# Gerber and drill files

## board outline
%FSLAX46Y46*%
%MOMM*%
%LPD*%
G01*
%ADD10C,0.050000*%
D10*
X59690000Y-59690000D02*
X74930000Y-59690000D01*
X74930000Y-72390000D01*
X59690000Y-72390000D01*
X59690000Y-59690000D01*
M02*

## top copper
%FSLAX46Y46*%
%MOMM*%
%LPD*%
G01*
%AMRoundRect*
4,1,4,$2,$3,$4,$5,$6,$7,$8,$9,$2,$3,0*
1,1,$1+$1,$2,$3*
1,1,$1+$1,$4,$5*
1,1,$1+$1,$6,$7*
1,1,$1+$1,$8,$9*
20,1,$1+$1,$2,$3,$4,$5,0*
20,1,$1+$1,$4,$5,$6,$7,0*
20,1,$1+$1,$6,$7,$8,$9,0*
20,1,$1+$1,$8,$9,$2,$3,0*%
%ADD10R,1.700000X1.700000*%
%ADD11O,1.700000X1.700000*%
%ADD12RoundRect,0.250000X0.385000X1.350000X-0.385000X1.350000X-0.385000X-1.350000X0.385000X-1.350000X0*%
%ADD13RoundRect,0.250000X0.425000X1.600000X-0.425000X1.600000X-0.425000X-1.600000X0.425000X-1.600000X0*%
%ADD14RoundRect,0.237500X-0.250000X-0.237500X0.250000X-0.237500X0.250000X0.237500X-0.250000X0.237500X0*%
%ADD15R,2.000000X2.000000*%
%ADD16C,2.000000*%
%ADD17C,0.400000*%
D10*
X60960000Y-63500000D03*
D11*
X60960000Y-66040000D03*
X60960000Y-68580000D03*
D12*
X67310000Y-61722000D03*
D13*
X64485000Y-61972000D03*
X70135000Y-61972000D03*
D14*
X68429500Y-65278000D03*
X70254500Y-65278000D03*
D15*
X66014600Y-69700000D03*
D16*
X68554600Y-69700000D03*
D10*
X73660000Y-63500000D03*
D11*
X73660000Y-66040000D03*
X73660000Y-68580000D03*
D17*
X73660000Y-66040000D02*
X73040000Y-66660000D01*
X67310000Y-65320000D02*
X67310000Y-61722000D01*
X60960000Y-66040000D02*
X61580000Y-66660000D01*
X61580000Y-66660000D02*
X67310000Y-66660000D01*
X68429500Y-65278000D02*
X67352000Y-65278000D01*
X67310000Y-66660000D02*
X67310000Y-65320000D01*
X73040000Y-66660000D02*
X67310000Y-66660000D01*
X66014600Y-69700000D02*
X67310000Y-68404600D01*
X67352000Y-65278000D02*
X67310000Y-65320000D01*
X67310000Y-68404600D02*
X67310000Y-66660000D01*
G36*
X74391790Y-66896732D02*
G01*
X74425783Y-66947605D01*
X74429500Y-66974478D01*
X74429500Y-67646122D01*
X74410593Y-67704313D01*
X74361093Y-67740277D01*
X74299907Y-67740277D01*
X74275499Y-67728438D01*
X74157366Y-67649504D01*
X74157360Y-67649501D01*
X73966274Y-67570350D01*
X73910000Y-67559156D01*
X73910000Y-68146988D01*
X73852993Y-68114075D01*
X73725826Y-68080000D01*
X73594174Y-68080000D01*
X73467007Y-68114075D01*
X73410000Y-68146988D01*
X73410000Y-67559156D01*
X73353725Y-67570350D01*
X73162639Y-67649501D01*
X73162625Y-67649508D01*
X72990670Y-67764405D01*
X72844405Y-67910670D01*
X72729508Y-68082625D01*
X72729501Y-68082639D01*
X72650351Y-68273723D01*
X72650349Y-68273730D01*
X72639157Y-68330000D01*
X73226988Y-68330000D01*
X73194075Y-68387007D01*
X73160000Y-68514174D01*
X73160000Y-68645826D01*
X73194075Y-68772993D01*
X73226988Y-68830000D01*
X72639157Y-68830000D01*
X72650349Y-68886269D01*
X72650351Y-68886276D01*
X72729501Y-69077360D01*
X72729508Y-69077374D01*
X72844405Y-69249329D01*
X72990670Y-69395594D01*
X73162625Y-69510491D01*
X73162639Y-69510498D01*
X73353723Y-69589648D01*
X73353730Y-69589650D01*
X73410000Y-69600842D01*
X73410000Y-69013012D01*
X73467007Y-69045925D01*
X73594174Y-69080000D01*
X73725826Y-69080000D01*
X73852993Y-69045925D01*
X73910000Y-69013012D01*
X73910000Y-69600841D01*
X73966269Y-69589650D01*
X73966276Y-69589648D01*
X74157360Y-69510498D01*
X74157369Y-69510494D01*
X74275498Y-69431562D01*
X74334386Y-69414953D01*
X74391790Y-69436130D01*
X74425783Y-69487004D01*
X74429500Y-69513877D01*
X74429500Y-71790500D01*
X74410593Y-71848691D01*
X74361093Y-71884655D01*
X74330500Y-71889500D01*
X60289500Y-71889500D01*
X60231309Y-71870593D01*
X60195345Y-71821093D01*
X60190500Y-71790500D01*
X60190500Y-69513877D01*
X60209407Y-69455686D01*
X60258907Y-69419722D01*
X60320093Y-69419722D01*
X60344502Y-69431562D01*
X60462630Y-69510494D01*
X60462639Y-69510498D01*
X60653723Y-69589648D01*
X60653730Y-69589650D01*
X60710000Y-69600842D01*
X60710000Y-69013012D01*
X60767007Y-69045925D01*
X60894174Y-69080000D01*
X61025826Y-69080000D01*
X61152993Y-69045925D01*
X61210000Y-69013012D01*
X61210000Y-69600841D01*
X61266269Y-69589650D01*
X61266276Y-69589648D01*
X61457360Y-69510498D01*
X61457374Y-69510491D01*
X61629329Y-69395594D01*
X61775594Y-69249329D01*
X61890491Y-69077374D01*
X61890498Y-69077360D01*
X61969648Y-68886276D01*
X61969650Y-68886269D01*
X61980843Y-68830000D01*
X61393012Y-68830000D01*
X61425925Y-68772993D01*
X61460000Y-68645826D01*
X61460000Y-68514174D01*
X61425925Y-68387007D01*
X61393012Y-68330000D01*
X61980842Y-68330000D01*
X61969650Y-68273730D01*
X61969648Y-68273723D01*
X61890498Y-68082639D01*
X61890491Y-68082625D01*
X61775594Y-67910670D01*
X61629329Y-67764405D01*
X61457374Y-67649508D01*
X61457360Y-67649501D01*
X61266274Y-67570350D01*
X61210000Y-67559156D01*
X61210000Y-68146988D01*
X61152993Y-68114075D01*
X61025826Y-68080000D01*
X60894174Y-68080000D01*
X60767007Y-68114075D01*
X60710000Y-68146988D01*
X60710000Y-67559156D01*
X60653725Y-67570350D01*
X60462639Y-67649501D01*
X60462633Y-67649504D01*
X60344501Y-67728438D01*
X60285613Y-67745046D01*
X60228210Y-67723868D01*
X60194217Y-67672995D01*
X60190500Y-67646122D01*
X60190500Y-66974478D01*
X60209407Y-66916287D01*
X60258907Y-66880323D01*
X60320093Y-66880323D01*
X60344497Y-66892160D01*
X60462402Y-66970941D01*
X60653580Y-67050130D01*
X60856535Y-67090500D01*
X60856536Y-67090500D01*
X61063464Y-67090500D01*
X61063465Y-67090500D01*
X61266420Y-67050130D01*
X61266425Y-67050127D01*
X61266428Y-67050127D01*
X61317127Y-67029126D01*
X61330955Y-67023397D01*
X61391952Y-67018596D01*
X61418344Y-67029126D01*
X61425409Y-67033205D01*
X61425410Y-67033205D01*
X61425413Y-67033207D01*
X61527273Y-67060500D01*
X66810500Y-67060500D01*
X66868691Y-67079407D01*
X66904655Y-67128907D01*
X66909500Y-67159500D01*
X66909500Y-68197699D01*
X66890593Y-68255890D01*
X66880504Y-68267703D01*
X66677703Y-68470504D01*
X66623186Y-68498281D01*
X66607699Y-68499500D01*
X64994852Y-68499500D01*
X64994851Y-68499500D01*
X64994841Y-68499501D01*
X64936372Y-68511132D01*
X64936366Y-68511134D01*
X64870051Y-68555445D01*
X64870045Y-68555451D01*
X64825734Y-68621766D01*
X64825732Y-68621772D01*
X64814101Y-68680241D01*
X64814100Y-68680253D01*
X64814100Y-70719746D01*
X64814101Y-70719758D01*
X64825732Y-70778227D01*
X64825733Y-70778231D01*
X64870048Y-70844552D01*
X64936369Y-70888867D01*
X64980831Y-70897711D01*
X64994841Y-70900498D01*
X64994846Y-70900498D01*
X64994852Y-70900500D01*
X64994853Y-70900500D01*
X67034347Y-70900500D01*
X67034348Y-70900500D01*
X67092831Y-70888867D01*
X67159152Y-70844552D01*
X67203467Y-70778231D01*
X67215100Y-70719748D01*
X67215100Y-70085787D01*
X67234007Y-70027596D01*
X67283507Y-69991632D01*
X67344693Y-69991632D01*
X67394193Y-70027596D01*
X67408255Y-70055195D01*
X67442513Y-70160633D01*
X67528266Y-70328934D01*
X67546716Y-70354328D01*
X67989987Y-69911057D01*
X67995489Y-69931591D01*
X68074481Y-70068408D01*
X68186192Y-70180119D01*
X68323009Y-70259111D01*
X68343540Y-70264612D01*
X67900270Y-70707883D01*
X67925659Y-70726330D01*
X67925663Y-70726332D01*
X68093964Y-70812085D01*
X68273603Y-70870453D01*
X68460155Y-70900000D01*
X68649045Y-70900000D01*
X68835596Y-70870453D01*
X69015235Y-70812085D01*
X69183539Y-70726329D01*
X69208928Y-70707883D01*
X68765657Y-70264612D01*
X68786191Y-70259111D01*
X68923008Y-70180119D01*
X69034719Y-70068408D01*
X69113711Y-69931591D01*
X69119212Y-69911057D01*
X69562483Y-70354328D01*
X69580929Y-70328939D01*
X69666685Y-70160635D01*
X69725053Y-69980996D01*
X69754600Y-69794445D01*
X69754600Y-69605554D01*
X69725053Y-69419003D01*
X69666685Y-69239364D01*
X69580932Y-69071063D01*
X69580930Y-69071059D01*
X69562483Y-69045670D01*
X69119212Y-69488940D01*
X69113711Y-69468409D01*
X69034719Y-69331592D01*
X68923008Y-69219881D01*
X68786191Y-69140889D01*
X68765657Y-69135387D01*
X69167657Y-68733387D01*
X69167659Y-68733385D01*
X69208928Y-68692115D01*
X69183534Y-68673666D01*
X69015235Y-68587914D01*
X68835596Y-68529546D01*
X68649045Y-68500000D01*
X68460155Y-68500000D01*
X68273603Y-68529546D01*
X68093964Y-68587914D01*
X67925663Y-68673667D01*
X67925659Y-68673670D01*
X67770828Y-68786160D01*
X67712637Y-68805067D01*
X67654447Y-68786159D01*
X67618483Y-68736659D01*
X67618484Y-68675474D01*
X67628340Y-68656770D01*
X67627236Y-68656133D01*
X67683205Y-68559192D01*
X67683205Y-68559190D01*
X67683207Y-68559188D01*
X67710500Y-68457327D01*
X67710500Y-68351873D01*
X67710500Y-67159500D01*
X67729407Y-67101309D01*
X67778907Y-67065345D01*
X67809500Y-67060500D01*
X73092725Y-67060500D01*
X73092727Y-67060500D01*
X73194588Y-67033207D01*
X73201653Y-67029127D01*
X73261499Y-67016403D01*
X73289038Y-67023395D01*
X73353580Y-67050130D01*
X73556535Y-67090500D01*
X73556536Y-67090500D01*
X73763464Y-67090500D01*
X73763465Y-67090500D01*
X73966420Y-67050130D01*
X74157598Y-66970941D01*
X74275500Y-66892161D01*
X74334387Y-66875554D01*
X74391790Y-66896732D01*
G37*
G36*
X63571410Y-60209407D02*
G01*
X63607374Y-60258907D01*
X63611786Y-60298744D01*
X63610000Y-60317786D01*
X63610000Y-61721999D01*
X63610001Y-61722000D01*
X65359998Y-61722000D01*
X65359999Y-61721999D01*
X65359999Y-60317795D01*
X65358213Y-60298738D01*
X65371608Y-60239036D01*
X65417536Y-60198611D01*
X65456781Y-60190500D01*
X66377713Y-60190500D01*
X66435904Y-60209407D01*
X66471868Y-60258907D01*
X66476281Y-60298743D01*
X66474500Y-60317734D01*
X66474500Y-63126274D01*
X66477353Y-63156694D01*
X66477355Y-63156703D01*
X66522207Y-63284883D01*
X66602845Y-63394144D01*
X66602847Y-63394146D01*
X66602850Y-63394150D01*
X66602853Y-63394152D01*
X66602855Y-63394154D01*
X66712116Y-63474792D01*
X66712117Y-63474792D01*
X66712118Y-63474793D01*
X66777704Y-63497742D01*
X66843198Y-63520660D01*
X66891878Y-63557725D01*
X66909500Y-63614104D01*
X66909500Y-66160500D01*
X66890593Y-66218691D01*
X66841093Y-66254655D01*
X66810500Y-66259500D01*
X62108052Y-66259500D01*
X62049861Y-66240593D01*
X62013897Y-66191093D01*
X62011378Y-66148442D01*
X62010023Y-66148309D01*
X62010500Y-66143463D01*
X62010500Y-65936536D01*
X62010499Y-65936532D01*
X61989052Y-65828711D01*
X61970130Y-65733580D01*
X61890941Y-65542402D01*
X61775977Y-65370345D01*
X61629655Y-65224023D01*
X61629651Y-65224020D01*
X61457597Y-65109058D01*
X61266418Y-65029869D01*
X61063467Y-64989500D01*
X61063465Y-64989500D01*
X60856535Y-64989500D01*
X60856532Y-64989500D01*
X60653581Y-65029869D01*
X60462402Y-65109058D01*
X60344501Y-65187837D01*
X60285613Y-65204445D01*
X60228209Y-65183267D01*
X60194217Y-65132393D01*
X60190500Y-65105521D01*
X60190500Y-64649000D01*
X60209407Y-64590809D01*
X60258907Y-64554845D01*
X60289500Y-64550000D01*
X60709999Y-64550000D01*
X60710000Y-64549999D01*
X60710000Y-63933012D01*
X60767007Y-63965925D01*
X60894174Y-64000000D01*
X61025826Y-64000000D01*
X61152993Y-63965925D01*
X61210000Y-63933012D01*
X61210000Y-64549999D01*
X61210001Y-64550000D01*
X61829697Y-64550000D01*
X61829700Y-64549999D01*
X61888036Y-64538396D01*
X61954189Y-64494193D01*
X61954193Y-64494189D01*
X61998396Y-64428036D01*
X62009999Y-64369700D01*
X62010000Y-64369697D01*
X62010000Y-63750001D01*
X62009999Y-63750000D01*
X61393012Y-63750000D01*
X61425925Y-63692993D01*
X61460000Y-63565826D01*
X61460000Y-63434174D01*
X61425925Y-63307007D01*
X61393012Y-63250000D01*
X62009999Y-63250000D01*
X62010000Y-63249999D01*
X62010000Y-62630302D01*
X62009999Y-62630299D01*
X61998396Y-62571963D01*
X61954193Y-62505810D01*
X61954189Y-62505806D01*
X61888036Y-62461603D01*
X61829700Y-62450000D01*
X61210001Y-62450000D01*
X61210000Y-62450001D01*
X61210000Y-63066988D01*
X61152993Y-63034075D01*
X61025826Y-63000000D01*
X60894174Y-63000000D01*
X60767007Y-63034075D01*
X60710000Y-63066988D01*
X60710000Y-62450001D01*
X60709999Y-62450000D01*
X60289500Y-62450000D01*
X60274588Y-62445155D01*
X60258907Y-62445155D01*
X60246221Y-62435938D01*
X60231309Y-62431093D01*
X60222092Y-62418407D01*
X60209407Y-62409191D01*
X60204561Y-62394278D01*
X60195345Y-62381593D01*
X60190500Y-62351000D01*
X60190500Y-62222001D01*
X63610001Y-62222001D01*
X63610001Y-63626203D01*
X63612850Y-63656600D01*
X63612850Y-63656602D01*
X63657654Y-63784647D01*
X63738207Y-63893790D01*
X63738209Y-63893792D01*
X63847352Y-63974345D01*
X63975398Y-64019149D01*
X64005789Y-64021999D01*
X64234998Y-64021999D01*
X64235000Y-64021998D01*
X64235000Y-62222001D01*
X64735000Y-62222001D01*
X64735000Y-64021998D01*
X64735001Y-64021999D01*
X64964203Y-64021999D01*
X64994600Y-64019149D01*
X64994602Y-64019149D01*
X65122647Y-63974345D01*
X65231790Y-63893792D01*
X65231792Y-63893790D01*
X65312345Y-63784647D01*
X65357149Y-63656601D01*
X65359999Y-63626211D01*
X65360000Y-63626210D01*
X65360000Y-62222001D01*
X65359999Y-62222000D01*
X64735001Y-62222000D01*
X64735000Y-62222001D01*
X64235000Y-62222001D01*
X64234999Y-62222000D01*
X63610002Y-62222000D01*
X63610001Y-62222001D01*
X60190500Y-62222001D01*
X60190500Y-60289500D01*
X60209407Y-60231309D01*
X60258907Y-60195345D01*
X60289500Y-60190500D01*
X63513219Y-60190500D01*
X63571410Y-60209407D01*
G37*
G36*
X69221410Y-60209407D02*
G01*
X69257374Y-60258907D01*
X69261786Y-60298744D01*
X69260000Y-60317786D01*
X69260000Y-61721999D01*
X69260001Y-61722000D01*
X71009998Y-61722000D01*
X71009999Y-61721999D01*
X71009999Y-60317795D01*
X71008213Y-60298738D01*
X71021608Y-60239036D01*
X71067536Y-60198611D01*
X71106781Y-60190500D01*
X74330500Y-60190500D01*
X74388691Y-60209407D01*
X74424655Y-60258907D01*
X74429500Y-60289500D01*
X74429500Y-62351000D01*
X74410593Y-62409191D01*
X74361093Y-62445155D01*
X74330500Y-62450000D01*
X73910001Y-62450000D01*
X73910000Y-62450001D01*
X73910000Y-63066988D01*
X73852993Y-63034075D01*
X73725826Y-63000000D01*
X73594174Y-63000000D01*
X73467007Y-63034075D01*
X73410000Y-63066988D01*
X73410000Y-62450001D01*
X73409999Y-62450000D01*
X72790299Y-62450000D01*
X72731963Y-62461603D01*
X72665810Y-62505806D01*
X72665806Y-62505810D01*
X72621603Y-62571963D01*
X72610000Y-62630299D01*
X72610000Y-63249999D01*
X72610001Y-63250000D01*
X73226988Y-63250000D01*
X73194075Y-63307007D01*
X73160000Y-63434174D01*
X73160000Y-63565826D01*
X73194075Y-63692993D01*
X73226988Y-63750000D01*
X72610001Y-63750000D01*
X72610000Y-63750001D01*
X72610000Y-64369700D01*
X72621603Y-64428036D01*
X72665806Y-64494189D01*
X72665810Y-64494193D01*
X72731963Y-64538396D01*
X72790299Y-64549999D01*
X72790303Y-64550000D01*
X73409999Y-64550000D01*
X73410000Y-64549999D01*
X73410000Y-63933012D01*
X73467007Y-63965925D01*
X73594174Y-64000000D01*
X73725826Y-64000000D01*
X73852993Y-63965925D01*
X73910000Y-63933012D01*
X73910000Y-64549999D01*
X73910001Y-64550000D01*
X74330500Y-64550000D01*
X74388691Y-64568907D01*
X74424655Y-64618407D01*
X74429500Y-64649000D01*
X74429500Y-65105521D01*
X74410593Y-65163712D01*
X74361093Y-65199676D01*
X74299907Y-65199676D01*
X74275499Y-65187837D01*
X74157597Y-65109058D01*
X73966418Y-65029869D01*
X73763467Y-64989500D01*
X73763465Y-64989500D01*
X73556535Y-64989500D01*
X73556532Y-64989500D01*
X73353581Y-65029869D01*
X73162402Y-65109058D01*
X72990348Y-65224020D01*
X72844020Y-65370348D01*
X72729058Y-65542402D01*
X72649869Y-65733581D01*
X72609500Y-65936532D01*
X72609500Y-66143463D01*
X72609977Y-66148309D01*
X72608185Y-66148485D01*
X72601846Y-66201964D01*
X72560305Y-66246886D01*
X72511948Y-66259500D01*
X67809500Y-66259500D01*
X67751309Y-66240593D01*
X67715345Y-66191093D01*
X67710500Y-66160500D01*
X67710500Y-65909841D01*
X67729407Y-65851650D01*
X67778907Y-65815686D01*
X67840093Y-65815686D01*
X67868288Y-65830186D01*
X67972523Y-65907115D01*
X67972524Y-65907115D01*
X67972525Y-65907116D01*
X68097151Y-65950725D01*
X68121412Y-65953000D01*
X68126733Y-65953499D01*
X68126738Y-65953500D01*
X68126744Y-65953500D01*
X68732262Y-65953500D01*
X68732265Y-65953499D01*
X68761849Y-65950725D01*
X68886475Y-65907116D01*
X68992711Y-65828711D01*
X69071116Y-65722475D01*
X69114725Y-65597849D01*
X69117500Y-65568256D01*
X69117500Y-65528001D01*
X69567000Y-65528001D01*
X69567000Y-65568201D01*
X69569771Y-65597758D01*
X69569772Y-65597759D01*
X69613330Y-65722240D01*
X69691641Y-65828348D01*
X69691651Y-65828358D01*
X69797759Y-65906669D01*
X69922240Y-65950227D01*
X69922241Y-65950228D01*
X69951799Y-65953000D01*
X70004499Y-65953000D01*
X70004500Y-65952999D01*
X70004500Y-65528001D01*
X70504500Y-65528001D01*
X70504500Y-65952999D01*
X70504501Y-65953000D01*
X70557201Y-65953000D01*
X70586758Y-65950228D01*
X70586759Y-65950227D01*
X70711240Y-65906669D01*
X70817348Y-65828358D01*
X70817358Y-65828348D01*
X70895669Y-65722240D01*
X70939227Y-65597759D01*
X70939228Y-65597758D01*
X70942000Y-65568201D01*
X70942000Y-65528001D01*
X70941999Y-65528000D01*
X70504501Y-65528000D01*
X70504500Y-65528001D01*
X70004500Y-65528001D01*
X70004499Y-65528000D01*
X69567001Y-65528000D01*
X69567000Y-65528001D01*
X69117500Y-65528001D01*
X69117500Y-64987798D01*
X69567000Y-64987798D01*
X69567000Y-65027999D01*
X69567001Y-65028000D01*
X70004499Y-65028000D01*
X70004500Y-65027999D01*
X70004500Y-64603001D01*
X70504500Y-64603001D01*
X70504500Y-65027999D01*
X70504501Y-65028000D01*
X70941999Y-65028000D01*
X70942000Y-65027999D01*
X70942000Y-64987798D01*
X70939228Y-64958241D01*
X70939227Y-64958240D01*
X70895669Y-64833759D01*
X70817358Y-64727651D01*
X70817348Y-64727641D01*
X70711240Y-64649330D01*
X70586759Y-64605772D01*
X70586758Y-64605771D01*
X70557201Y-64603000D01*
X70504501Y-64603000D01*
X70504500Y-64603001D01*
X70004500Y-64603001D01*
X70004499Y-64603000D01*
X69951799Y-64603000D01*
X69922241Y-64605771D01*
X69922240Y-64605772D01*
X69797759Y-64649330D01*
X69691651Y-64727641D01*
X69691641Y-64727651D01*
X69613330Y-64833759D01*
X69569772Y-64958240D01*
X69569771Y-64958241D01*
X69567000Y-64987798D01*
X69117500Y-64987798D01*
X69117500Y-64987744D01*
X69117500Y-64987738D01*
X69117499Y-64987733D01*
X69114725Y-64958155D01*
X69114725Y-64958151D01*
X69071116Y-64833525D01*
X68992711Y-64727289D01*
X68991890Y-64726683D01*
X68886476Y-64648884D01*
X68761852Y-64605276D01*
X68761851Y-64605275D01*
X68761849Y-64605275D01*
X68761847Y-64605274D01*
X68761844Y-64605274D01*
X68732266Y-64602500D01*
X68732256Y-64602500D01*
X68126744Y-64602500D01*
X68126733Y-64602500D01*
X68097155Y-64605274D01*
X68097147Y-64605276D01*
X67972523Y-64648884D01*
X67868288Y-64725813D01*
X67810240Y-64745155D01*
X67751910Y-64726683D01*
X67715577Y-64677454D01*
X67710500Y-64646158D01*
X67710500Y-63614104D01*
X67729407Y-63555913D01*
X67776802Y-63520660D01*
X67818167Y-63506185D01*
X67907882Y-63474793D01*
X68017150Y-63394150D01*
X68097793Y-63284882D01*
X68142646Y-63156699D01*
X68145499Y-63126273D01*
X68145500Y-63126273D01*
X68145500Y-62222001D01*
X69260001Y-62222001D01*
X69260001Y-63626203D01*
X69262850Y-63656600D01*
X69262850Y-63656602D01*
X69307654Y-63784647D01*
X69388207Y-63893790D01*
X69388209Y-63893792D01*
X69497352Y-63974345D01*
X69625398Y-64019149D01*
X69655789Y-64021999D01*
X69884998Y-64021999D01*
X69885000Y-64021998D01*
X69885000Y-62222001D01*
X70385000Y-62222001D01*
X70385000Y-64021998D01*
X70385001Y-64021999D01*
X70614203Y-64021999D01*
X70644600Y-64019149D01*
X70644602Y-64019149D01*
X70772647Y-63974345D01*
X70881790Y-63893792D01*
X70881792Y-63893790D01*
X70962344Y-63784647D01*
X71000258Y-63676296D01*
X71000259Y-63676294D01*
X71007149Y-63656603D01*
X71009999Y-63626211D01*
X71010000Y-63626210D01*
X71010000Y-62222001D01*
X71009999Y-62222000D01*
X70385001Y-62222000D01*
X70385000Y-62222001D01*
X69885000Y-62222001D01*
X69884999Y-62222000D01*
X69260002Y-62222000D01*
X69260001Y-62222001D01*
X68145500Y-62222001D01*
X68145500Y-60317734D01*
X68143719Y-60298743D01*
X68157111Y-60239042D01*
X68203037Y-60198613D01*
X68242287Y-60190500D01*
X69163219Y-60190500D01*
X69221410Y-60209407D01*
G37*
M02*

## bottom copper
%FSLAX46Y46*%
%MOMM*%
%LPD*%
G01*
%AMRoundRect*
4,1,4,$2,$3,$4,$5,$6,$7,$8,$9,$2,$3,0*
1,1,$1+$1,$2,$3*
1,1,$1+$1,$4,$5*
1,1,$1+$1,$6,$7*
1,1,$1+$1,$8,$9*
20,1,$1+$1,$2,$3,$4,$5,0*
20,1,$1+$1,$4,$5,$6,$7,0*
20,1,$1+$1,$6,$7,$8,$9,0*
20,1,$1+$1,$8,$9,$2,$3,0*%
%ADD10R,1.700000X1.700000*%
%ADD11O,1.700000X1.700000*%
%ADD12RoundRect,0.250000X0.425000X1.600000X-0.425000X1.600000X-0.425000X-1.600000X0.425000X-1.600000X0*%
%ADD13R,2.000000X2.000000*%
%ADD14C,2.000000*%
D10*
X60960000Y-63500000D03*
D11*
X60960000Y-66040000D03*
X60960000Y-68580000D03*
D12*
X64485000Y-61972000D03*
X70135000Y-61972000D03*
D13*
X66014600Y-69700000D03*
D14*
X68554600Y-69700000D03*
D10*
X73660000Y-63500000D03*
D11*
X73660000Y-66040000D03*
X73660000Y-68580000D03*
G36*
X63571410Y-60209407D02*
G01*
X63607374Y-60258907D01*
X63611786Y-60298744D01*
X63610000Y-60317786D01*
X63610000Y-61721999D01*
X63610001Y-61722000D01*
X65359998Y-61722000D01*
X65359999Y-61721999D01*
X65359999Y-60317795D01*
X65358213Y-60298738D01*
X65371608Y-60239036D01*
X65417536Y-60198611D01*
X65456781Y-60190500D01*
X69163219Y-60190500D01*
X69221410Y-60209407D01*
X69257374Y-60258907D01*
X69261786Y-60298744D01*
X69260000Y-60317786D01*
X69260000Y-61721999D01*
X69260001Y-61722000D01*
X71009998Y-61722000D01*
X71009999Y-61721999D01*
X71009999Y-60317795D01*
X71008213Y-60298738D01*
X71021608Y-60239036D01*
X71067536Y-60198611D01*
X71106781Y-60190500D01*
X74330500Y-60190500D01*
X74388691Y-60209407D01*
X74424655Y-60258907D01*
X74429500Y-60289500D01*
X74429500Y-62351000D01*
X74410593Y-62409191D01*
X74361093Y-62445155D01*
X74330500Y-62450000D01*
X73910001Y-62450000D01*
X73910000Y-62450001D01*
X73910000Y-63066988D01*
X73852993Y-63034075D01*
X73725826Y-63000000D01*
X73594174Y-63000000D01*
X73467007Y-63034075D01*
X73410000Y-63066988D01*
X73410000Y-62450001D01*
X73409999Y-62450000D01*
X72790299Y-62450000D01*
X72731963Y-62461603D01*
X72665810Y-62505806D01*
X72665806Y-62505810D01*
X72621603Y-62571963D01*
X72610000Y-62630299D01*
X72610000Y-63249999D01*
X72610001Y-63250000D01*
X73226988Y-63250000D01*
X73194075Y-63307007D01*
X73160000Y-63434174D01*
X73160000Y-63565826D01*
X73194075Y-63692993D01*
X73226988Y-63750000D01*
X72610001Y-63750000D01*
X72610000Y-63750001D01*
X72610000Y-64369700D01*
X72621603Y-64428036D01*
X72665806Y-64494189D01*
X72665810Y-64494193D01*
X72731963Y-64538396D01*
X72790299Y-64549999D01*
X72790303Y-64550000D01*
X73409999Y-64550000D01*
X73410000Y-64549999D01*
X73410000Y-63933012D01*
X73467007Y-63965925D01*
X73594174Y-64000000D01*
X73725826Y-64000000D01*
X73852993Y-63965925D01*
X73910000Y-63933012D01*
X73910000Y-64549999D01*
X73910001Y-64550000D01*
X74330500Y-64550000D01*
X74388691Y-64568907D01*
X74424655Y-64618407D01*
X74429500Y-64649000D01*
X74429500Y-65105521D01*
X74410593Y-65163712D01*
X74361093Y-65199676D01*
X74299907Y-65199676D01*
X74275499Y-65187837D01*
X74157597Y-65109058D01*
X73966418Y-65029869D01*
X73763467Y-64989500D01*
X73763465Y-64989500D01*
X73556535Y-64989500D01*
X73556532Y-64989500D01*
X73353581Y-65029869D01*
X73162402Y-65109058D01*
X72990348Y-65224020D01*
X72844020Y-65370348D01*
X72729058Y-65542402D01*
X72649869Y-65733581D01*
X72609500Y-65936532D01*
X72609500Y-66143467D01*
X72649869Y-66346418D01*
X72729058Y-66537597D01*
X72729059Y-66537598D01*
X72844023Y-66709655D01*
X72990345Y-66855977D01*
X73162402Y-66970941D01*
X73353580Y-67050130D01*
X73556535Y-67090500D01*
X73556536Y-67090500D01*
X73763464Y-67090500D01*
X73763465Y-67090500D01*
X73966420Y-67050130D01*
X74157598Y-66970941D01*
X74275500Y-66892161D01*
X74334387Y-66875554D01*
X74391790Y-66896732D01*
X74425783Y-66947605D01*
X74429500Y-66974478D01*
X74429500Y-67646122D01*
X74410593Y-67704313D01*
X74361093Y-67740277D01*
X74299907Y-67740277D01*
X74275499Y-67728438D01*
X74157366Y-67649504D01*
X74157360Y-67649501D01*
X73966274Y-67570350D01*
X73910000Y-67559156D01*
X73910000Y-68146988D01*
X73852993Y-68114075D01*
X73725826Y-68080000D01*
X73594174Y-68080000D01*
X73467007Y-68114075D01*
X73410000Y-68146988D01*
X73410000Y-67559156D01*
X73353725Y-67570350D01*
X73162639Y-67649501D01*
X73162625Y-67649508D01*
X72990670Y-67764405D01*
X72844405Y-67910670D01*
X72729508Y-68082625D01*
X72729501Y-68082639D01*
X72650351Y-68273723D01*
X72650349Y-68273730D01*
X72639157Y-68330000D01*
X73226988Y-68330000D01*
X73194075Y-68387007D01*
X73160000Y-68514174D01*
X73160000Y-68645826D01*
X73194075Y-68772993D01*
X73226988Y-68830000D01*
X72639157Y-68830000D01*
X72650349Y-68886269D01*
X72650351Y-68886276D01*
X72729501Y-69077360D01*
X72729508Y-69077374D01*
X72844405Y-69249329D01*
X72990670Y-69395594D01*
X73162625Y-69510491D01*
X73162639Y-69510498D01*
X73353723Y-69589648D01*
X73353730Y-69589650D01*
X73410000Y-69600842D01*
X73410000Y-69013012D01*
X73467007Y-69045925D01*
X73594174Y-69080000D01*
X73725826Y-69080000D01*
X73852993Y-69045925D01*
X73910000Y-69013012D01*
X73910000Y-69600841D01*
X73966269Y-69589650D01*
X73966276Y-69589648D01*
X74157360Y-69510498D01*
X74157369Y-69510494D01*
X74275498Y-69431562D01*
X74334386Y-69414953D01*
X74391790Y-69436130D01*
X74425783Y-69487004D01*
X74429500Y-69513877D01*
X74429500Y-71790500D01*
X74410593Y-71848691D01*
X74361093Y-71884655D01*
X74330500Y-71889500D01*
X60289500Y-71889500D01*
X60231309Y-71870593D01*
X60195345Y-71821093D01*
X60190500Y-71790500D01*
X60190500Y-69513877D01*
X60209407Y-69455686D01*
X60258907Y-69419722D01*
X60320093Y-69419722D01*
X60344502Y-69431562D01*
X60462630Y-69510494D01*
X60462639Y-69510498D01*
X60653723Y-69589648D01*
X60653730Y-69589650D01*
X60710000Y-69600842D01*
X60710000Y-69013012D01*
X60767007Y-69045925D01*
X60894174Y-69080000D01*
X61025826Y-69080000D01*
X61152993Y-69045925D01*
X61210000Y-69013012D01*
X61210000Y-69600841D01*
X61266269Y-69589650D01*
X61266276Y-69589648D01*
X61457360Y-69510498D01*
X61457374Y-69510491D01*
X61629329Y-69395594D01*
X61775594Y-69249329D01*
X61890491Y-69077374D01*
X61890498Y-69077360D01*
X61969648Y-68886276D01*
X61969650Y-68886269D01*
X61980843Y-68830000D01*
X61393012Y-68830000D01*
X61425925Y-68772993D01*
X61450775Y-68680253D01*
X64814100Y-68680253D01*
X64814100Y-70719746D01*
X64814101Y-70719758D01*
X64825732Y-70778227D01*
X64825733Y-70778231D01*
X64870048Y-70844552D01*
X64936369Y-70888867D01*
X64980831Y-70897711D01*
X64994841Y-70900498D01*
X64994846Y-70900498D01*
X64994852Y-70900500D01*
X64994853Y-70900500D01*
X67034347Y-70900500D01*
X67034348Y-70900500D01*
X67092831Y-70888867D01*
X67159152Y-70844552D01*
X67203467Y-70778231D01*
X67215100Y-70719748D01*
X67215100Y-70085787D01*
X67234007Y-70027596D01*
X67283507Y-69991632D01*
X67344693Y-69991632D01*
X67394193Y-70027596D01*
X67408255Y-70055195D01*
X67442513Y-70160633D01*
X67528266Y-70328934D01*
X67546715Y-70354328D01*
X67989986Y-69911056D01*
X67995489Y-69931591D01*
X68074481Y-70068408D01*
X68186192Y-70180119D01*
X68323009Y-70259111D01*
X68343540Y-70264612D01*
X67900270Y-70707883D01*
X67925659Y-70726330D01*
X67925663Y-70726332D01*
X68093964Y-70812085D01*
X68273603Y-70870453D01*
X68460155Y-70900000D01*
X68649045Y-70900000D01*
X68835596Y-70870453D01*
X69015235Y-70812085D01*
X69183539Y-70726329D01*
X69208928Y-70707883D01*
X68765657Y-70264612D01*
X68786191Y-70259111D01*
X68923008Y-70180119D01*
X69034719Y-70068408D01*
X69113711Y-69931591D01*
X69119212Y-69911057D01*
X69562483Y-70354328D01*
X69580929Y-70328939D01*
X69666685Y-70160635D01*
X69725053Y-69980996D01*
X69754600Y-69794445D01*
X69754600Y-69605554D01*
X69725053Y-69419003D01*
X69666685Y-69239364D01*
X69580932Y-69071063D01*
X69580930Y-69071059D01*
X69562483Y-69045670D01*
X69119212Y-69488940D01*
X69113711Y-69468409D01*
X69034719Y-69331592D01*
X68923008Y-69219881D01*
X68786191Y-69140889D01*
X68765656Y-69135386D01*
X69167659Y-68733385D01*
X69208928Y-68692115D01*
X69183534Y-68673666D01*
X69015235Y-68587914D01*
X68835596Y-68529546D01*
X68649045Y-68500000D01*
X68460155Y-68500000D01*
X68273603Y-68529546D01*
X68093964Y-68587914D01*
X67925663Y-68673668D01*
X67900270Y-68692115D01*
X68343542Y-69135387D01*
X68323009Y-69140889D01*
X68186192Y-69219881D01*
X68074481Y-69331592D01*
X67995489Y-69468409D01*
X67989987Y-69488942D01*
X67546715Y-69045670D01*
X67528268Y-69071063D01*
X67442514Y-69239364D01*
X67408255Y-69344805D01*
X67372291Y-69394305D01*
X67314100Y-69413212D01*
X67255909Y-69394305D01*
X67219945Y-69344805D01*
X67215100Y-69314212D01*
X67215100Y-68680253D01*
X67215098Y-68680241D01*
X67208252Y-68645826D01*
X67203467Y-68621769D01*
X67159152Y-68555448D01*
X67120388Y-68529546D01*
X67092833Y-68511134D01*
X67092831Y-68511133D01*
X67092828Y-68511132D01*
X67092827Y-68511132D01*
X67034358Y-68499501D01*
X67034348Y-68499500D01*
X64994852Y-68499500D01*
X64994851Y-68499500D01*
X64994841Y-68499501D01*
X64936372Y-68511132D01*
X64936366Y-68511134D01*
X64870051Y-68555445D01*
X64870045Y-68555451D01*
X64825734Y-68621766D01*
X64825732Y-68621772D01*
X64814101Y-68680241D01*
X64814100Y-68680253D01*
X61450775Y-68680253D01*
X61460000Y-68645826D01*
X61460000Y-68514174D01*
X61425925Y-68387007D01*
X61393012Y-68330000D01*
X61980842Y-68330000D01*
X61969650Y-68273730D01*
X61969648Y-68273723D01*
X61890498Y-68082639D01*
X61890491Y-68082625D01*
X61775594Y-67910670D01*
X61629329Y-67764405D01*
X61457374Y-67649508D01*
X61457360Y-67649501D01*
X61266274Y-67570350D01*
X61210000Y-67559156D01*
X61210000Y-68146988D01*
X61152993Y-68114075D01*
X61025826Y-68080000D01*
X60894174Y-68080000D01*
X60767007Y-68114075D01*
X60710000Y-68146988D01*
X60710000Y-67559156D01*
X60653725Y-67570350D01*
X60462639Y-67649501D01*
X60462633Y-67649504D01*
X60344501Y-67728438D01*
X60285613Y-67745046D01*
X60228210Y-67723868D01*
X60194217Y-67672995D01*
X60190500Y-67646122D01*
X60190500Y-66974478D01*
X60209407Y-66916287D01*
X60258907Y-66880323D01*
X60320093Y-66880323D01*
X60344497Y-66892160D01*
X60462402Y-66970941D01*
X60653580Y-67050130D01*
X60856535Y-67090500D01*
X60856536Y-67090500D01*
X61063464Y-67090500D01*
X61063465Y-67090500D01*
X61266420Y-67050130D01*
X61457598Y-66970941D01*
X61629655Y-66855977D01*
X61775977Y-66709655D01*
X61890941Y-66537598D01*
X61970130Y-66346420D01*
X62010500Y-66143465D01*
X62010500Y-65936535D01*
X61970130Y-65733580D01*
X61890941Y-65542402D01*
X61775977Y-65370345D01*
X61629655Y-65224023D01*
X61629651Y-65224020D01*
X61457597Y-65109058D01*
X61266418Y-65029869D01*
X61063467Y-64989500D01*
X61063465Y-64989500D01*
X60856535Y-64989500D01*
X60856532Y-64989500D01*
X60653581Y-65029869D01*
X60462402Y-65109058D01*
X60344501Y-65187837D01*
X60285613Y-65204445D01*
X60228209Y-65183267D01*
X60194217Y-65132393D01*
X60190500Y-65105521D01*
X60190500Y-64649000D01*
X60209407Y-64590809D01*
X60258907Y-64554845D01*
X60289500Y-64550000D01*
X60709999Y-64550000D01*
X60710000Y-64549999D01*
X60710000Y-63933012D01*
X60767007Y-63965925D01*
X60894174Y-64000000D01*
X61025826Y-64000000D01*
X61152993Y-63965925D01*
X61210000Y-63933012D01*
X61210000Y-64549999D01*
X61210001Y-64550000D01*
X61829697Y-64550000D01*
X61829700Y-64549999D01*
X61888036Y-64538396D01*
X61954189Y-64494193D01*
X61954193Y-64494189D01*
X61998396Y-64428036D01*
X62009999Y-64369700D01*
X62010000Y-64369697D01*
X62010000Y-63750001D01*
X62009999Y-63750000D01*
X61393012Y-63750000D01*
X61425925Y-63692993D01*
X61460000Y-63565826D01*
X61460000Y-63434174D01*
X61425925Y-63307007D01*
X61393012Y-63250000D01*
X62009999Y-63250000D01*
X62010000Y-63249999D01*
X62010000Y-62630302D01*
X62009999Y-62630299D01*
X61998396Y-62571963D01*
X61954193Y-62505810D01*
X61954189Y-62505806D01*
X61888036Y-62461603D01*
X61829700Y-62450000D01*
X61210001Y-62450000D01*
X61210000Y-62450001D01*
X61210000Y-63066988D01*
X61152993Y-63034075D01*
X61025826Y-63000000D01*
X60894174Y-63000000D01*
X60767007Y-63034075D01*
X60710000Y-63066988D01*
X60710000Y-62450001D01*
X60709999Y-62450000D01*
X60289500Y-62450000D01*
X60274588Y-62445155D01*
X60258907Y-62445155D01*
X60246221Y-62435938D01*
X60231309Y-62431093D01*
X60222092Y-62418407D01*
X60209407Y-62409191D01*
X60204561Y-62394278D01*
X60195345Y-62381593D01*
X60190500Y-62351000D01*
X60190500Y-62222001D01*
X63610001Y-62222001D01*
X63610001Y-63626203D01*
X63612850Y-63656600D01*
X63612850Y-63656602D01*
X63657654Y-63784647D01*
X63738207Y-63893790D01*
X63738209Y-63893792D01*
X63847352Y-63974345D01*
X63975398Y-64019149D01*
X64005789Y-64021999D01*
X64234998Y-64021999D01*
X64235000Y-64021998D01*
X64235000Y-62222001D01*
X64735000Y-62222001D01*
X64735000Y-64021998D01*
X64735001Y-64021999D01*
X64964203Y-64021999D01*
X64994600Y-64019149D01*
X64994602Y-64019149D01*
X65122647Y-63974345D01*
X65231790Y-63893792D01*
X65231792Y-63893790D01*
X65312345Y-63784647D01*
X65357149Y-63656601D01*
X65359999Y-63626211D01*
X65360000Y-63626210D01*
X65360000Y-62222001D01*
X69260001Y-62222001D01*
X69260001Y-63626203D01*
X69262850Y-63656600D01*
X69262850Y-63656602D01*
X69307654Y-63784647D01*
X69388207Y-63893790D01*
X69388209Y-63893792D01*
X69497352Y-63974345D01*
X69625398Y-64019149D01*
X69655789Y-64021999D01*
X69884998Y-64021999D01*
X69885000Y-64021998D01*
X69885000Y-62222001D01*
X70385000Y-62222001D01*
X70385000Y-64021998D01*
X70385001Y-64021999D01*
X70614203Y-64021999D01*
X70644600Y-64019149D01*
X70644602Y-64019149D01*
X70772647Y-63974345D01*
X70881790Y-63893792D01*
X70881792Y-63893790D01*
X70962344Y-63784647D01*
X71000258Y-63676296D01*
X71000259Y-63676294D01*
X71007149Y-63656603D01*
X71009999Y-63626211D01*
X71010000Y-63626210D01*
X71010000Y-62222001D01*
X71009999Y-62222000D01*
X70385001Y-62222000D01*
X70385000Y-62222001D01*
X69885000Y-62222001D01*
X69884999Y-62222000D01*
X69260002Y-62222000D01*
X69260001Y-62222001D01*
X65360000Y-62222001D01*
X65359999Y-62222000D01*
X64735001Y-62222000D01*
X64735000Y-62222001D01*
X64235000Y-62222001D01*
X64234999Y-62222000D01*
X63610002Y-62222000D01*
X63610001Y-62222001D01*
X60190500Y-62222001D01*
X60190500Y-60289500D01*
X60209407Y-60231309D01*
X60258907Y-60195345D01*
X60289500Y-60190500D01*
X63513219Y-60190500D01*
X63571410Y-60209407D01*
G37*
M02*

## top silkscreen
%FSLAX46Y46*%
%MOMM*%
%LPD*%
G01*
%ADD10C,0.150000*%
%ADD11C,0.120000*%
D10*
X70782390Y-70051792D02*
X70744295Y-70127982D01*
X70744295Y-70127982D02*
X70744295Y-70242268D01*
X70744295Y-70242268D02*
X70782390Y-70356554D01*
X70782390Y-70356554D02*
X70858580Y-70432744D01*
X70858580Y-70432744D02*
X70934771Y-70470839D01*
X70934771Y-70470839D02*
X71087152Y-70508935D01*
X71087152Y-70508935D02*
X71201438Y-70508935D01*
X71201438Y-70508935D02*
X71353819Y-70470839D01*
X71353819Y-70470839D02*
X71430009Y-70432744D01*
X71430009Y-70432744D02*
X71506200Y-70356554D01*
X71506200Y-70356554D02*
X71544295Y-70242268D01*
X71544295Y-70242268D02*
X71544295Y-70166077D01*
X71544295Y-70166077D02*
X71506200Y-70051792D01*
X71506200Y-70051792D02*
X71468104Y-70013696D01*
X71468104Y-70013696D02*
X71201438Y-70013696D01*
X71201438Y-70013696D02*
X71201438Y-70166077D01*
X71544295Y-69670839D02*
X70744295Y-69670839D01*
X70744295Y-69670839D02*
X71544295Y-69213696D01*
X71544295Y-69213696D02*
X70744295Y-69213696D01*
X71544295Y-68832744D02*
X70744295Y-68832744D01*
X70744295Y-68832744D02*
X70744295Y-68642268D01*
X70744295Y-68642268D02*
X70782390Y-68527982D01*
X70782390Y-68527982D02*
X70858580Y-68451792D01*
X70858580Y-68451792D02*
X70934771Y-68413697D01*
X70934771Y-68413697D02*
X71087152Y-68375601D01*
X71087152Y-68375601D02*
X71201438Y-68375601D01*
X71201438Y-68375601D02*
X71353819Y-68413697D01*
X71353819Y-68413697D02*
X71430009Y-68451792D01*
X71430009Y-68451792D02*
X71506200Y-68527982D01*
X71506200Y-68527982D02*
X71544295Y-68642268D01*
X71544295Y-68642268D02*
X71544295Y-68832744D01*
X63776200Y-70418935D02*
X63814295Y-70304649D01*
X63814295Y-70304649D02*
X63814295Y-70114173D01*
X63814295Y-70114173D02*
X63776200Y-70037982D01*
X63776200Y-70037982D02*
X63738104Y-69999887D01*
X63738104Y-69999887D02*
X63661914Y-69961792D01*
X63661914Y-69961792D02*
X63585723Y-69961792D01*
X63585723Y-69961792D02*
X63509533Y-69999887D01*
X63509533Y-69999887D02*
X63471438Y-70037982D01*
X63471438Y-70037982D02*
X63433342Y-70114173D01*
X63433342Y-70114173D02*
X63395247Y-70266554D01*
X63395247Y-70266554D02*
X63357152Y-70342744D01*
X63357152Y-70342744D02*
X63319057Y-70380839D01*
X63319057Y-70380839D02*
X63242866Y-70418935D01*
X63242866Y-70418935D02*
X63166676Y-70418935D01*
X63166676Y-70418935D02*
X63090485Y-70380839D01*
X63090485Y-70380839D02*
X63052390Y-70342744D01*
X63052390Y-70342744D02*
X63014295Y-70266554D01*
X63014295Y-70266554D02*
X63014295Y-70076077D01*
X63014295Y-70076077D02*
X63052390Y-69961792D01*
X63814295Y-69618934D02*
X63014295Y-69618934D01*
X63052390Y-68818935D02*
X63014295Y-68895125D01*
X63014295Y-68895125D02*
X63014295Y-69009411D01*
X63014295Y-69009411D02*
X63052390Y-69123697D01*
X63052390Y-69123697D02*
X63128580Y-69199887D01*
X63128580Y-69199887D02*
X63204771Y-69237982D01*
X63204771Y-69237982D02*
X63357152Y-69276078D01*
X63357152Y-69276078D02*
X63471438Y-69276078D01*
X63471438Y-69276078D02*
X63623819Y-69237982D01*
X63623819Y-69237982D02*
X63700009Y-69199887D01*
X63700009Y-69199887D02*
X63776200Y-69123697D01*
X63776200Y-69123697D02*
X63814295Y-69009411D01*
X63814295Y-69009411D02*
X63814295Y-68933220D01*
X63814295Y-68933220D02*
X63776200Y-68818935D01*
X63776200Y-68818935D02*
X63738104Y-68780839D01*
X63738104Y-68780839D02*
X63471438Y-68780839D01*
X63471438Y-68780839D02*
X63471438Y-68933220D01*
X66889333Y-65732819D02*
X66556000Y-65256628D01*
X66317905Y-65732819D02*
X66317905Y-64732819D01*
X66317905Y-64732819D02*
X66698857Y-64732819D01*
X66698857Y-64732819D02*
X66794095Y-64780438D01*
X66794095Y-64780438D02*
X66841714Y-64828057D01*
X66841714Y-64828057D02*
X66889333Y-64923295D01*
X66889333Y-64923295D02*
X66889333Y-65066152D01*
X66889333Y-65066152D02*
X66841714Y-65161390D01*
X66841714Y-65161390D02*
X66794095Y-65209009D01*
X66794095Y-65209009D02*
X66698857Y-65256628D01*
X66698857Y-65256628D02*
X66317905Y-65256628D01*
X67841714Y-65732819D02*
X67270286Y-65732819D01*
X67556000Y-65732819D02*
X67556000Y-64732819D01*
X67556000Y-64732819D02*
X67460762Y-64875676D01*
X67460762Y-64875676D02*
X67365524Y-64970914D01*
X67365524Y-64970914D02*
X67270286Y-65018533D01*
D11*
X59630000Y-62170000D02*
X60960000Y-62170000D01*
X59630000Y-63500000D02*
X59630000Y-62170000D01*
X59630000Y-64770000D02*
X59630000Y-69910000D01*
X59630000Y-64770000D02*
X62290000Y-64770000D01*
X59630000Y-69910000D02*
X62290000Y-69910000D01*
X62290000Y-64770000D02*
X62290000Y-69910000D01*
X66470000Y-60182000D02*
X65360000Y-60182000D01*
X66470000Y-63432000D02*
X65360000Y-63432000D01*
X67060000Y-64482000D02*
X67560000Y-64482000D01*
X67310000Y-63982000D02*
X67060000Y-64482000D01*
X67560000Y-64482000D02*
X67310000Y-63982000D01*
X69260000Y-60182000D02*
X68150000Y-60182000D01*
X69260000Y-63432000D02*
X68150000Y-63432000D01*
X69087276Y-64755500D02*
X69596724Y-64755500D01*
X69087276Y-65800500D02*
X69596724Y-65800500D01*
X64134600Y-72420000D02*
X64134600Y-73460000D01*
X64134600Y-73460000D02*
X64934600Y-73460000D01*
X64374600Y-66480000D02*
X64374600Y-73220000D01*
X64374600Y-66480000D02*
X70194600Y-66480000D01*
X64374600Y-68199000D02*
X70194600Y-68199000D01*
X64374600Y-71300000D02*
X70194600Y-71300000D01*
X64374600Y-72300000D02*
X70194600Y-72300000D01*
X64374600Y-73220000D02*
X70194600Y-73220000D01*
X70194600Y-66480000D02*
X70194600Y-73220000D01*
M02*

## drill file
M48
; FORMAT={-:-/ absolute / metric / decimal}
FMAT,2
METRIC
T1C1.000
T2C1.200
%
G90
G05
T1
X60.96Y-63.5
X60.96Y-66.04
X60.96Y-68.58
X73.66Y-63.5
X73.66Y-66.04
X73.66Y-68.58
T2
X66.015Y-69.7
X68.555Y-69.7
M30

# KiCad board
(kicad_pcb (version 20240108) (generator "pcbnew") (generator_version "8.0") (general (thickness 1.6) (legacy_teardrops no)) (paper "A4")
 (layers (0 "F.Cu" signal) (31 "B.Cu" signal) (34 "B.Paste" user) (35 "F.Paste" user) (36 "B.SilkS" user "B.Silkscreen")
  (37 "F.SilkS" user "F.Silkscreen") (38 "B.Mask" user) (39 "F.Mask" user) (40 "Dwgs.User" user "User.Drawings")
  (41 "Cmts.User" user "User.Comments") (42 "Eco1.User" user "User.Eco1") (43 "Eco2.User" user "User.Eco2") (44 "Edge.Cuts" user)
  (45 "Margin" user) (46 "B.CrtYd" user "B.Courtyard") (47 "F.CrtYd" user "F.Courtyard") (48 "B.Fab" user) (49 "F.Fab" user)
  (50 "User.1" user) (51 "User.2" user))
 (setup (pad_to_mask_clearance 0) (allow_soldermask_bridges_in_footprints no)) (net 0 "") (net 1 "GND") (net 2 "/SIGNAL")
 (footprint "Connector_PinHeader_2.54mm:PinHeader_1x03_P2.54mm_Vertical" (layer "F.Cu") (at 60.96 63.5)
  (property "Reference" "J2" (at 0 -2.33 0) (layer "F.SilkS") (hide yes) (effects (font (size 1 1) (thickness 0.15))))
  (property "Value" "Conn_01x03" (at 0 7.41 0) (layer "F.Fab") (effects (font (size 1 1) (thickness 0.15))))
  (fp_line (start -1.33 -1.33) (end 0 -1.33) (stroke (width 0.12) (type solid)) (layer "F.SilkS"))
  (fp_line (start -1.33 0) (end -1.33 -1.33) (stroke (width 0.12) (type solid)) (layer "F.SilkS"))
  (fp_line (start -1.33 1.27) (end -1.33 6.41) (stroke (width 0.12) (type solid)) (layer "F.SilkS"))
  (fp_line (start -1.33 1.27) (end 1.33 1.27) (stroke (width 0.12) (type solid)) (layer "F.SilkS"))
  (fp_line (start -1.33 6.41) (end 1.33 6.41) (stroke (width 0.12) (type solid)) (layer "F.SilkS"))
  (fp_line (start 1.33 1.27) (end 1.33 6.41) (stroke (width 0.12) (type solid)) (layer "F.SilkS"))
  (pad "1" thru_hole rect (at 0 0) (size 1.7 1.7) (drill 1) (layers "*.Cu" "*.Mask") (remove_unused_layers no) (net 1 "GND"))
  (pad "2" thru_hole oval (at 0 2.54) (size 1.7 1.7) (drill 1) (layers "*.Cu" "*.Mask") (remove_unused_layers no) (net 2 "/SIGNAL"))
  (pad "3" thru_hole oval (at 0 5.08) (size 1.7 1.7) (drill 1) (layers "*.Cu" "*.Mask") (remove_unused_layers no) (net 1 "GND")))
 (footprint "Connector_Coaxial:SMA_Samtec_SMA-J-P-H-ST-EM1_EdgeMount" (layer "F.Cu") (at 67.31 61.722 90)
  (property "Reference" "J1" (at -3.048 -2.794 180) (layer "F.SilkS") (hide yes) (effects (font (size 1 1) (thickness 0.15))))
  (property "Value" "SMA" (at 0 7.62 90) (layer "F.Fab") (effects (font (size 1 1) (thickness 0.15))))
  (fp_line (start 1.54 -0.84) (end 1.54 -1.95) (stroke (width 0.12) (type solid)) (layer "F.SilkS"))
  (fp_line (start -1.71 -0.84) (end -1.71 -1.95) (stroke (width 0.12) (type solid)) (layer "F.SilkS"))
  (fp_line (start -2.76 -0.25) (end -2.76 0.25) (stroke (width 0.12) (type solid)) (layer "F.SilkS"))
  (fp_line (start -2.26 0) (end -2.76 -0.25) (stroke (width 0.12) (type solid)) (layer "F.SilkS"))
  (fp_line (start -2.76 0.25) (end -2.26 0) (stroke (width 0.12) (type solid)) (layer "F.SilkS"))
  (fp_line (start 1.54 1.95) (end 1.54 0.84) (stroke (width 0.12) (type solid)) (layer "F.SilkS"))
  (fp_line (start -1.71 1.95) (end -1.71 0.84) (stroke (width 0.12) (type solid)) (layer "F.SilkS"))
  (pad "1" smd roundrect (at 0 0 180) (size 1.27 3.2) (layers "F.Cu" "F.Mask") (roundrect_rratio 0.1968503937) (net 2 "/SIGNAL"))
  (pad "2" smd roundrect (at -0.25 -2.825 180) (size 1.35 3.7) (layers "F.Cu" "F.Mask") (roundrect_rratio 0.1851851852) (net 1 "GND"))
  (pad "2" smd roundrect (at -0.25 -2.825 180) (size 1.35 3.7) (layers "B.Cu" "B.Mask") (roundrect_rratio 0.1851851852) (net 1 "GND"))
  (pad "2" smd roundrect (at -0.25 2.825 180) (size 1.35 3.7) (layers "F.Cu" "F.Mask") (roundrect_rratio 0.1851851852) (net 1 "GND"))
  (pad "2" smd roundrect (at -0.25 2.825 180) (size 1.35 3.7) (layers "B.Cu" "B.Mask") (roundrect_rratio 0.1851851852) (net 1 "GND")))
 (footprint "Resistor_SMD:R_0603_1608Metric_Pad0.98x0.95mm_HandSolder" (layer "F.Cu") (at 69.342 65.278)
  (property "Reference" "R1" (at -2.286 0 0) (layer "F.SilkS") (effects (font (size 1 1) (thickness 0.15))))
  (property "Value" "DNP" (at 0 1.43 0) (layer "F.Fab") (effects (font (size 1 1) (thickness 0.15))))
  (fp_line (start -0.254724 -0.5225) (end 0.254724 -0.5225) (stroke (width 0.12) (type solid)) (layer "F.SilkS"))
  (fp_line (start -0.254724 0.5225) (end 0.254724 0.5225) (stroke (width 0.12) (type solid)) (layer "F.SilkS"))
  (pad "1" smd roundrect (at -0.9125 0) (size 0.975 0.95) (layers "F.Cu" "F.Paste" "F.Mask") (roundrect_rratio 0.25) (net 2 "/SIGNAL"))
  (pad "2" smd roundrect (at 0.9125 0) (size 0.975 0.95) (layers "F.Cu" "F.Paste" "F.Mask") (roundrect_rratio 0.25) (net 1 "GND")))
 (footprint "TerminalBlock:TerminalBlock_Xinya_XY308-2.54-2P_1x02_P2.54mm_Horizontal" (layer "F.Cu") (at 66.0146 69.7)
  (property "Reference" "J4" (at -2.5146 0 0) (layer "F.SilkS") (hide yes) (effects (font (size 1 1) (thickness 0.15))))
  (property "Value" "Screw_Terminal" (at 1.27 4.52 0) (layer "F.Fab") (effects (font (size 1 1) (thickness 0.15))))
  (fp_line (start -1.88 2.72) (end -1.88 3.76) (stroke (width 0.12) (type solid)) (layer "F.SilkS"))
  (fp_line (start -1.88 3.76) (end -1.08 3.76) (stroke (width 0.12) (type solid)) (layer "F.SilkS"))
  (fp_line (start -1.64 -3.22) (end -1.64 3.52) (stroke (width 0.12) (type solid)) (layer "F.SilkS"))
  (fp_line (start -1.64 -3.22) (end 4.18 -3.22) (stroke (width 0.12) (type solid)) (layer "F.SilkS"))
  (fp_line (start -1.64 -1.501) (end 4.18 -1.501) (stroke (width 0.12) (type solid)) (layer "F.SilkS"))
  (fp_line (start -1.64 1.6) (end 4.18 1.6) (stroke (width 0.12) (type solid)) (layer "F.SilkS"))
  (fp_line (start -1.64 2.6) (end 4.18 2.6) (stroke (width 0.12) (type solid)) (layer "F.SilkS"))
  (fp_line (start -1.64 3.52) (end 4.18 3.52) (stroke (width 0.12) (type solid)) (layer "F.SilkS"))
  (fp_line (start 4.18 -3.22) (end 4.18 3.52) (stroke (width 0.12) (type solid)) (layer "F.SilkS"))
  (pad "1" thru_hole rect (at 0 0) (size 2 2) (drill 1.2) (layers "*.Cu" "*.Mask") (remove_unused_layers no) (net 2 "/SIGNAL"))
  (pad "2" thru_hole circle (at 2.54 0) (size 2 2) (drill 1.2) (layers "*.Cu" "*.Mask") (remove_unused_layers no) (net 1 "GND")))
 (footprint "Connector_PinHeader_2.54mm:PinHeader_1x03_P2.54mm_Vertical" (layer "B.Cu") (at 73.66 63.5 180)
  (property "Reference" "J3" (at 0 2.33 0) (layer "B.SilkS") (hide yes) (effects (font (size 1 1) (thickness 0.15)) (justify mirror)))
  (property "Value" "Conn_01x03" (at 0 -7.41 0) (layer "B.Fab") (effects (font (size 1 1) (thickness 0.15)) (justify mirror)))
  (pad "1" thru_hole rect (at 0 0 180) (size 1.7 1.7) (drill 1) (layers "*.Cu" "*.Mask") (remove_unused_layers no) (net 1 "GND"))
  (pad "2" thru_hole oval (at 0 -2.54 180) (size 1.7 1.7) (drill 1) (layers "*.Cu" "*.Mask") (remove_unused_layers no) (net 2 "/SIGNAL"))
  (pad "3" thru_hole oval (at 0 -5.08 180) (size 1.7 1.7) (drill 1) (layers "*.Cu" "*.Mask") (remove_unused_layers no) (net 1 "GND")))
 (gr_rect (start 59.69 59.69) (end 74.93 72.39) (stroke (width 0.05) (type default)) (fill none) (layer "Edge.Cuts"))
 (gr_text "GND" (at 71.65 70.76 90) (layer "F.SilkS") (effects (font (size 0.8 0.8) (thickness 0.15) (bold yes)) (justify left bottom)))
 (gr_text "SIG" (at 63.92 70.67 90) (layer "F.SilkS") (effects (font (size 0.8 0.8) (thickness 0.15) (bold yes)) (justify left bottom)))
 (segment (start 73.66 66.04) (end 73.04 66.66) (width 0.4) (layer "F.Cu") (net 2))
 (segment (start 67.31 65.32) (end 67.31 61.722) (width 0.4) (layer "F.Cu") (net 2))
 (segment (start 60.96 66.04) (end 61.58 66.66) (width 0.4) (layer "F.Cu") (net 2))
 (segment (start 61.58 66.66) (end 67.31 66.66) (width 0.4) (layer "F.Cu") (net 2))
 (segment (start 68.4295 65.278) (end 67.352 65.278) (width 0.4) (layer "F.Cu") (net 2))
 (segment (start 67.31 66.66) (end 67.31 65.32) (width 0.4) (layer "F.Cu") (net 2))
 (segment (start 73.04 66.66) (end 67.31 66.66) (width 0.4) (layer "F.Cu") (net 2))
 (segment (start 66.0146 69.7) (end 67.31 68.4046) (width 0.4) (layer "F.Cu") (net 2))
 (segment (start 67.352 65.278) (end 67.31 65.32) (width 0.4) (layer "F.Cu") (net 2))
 (segment (start 67.31 68.4046) (end 67.31 66.66) (width 0.4) (layer "F.Cu") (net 2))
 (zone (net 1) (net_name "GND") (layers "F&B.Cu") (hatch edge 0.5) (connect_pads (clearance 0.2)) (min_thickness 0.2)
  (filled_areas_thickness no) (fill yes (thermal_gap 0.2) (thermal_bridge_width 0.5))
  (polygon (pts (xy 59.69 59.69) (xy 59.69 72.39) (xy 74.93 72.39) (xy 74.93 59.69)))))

